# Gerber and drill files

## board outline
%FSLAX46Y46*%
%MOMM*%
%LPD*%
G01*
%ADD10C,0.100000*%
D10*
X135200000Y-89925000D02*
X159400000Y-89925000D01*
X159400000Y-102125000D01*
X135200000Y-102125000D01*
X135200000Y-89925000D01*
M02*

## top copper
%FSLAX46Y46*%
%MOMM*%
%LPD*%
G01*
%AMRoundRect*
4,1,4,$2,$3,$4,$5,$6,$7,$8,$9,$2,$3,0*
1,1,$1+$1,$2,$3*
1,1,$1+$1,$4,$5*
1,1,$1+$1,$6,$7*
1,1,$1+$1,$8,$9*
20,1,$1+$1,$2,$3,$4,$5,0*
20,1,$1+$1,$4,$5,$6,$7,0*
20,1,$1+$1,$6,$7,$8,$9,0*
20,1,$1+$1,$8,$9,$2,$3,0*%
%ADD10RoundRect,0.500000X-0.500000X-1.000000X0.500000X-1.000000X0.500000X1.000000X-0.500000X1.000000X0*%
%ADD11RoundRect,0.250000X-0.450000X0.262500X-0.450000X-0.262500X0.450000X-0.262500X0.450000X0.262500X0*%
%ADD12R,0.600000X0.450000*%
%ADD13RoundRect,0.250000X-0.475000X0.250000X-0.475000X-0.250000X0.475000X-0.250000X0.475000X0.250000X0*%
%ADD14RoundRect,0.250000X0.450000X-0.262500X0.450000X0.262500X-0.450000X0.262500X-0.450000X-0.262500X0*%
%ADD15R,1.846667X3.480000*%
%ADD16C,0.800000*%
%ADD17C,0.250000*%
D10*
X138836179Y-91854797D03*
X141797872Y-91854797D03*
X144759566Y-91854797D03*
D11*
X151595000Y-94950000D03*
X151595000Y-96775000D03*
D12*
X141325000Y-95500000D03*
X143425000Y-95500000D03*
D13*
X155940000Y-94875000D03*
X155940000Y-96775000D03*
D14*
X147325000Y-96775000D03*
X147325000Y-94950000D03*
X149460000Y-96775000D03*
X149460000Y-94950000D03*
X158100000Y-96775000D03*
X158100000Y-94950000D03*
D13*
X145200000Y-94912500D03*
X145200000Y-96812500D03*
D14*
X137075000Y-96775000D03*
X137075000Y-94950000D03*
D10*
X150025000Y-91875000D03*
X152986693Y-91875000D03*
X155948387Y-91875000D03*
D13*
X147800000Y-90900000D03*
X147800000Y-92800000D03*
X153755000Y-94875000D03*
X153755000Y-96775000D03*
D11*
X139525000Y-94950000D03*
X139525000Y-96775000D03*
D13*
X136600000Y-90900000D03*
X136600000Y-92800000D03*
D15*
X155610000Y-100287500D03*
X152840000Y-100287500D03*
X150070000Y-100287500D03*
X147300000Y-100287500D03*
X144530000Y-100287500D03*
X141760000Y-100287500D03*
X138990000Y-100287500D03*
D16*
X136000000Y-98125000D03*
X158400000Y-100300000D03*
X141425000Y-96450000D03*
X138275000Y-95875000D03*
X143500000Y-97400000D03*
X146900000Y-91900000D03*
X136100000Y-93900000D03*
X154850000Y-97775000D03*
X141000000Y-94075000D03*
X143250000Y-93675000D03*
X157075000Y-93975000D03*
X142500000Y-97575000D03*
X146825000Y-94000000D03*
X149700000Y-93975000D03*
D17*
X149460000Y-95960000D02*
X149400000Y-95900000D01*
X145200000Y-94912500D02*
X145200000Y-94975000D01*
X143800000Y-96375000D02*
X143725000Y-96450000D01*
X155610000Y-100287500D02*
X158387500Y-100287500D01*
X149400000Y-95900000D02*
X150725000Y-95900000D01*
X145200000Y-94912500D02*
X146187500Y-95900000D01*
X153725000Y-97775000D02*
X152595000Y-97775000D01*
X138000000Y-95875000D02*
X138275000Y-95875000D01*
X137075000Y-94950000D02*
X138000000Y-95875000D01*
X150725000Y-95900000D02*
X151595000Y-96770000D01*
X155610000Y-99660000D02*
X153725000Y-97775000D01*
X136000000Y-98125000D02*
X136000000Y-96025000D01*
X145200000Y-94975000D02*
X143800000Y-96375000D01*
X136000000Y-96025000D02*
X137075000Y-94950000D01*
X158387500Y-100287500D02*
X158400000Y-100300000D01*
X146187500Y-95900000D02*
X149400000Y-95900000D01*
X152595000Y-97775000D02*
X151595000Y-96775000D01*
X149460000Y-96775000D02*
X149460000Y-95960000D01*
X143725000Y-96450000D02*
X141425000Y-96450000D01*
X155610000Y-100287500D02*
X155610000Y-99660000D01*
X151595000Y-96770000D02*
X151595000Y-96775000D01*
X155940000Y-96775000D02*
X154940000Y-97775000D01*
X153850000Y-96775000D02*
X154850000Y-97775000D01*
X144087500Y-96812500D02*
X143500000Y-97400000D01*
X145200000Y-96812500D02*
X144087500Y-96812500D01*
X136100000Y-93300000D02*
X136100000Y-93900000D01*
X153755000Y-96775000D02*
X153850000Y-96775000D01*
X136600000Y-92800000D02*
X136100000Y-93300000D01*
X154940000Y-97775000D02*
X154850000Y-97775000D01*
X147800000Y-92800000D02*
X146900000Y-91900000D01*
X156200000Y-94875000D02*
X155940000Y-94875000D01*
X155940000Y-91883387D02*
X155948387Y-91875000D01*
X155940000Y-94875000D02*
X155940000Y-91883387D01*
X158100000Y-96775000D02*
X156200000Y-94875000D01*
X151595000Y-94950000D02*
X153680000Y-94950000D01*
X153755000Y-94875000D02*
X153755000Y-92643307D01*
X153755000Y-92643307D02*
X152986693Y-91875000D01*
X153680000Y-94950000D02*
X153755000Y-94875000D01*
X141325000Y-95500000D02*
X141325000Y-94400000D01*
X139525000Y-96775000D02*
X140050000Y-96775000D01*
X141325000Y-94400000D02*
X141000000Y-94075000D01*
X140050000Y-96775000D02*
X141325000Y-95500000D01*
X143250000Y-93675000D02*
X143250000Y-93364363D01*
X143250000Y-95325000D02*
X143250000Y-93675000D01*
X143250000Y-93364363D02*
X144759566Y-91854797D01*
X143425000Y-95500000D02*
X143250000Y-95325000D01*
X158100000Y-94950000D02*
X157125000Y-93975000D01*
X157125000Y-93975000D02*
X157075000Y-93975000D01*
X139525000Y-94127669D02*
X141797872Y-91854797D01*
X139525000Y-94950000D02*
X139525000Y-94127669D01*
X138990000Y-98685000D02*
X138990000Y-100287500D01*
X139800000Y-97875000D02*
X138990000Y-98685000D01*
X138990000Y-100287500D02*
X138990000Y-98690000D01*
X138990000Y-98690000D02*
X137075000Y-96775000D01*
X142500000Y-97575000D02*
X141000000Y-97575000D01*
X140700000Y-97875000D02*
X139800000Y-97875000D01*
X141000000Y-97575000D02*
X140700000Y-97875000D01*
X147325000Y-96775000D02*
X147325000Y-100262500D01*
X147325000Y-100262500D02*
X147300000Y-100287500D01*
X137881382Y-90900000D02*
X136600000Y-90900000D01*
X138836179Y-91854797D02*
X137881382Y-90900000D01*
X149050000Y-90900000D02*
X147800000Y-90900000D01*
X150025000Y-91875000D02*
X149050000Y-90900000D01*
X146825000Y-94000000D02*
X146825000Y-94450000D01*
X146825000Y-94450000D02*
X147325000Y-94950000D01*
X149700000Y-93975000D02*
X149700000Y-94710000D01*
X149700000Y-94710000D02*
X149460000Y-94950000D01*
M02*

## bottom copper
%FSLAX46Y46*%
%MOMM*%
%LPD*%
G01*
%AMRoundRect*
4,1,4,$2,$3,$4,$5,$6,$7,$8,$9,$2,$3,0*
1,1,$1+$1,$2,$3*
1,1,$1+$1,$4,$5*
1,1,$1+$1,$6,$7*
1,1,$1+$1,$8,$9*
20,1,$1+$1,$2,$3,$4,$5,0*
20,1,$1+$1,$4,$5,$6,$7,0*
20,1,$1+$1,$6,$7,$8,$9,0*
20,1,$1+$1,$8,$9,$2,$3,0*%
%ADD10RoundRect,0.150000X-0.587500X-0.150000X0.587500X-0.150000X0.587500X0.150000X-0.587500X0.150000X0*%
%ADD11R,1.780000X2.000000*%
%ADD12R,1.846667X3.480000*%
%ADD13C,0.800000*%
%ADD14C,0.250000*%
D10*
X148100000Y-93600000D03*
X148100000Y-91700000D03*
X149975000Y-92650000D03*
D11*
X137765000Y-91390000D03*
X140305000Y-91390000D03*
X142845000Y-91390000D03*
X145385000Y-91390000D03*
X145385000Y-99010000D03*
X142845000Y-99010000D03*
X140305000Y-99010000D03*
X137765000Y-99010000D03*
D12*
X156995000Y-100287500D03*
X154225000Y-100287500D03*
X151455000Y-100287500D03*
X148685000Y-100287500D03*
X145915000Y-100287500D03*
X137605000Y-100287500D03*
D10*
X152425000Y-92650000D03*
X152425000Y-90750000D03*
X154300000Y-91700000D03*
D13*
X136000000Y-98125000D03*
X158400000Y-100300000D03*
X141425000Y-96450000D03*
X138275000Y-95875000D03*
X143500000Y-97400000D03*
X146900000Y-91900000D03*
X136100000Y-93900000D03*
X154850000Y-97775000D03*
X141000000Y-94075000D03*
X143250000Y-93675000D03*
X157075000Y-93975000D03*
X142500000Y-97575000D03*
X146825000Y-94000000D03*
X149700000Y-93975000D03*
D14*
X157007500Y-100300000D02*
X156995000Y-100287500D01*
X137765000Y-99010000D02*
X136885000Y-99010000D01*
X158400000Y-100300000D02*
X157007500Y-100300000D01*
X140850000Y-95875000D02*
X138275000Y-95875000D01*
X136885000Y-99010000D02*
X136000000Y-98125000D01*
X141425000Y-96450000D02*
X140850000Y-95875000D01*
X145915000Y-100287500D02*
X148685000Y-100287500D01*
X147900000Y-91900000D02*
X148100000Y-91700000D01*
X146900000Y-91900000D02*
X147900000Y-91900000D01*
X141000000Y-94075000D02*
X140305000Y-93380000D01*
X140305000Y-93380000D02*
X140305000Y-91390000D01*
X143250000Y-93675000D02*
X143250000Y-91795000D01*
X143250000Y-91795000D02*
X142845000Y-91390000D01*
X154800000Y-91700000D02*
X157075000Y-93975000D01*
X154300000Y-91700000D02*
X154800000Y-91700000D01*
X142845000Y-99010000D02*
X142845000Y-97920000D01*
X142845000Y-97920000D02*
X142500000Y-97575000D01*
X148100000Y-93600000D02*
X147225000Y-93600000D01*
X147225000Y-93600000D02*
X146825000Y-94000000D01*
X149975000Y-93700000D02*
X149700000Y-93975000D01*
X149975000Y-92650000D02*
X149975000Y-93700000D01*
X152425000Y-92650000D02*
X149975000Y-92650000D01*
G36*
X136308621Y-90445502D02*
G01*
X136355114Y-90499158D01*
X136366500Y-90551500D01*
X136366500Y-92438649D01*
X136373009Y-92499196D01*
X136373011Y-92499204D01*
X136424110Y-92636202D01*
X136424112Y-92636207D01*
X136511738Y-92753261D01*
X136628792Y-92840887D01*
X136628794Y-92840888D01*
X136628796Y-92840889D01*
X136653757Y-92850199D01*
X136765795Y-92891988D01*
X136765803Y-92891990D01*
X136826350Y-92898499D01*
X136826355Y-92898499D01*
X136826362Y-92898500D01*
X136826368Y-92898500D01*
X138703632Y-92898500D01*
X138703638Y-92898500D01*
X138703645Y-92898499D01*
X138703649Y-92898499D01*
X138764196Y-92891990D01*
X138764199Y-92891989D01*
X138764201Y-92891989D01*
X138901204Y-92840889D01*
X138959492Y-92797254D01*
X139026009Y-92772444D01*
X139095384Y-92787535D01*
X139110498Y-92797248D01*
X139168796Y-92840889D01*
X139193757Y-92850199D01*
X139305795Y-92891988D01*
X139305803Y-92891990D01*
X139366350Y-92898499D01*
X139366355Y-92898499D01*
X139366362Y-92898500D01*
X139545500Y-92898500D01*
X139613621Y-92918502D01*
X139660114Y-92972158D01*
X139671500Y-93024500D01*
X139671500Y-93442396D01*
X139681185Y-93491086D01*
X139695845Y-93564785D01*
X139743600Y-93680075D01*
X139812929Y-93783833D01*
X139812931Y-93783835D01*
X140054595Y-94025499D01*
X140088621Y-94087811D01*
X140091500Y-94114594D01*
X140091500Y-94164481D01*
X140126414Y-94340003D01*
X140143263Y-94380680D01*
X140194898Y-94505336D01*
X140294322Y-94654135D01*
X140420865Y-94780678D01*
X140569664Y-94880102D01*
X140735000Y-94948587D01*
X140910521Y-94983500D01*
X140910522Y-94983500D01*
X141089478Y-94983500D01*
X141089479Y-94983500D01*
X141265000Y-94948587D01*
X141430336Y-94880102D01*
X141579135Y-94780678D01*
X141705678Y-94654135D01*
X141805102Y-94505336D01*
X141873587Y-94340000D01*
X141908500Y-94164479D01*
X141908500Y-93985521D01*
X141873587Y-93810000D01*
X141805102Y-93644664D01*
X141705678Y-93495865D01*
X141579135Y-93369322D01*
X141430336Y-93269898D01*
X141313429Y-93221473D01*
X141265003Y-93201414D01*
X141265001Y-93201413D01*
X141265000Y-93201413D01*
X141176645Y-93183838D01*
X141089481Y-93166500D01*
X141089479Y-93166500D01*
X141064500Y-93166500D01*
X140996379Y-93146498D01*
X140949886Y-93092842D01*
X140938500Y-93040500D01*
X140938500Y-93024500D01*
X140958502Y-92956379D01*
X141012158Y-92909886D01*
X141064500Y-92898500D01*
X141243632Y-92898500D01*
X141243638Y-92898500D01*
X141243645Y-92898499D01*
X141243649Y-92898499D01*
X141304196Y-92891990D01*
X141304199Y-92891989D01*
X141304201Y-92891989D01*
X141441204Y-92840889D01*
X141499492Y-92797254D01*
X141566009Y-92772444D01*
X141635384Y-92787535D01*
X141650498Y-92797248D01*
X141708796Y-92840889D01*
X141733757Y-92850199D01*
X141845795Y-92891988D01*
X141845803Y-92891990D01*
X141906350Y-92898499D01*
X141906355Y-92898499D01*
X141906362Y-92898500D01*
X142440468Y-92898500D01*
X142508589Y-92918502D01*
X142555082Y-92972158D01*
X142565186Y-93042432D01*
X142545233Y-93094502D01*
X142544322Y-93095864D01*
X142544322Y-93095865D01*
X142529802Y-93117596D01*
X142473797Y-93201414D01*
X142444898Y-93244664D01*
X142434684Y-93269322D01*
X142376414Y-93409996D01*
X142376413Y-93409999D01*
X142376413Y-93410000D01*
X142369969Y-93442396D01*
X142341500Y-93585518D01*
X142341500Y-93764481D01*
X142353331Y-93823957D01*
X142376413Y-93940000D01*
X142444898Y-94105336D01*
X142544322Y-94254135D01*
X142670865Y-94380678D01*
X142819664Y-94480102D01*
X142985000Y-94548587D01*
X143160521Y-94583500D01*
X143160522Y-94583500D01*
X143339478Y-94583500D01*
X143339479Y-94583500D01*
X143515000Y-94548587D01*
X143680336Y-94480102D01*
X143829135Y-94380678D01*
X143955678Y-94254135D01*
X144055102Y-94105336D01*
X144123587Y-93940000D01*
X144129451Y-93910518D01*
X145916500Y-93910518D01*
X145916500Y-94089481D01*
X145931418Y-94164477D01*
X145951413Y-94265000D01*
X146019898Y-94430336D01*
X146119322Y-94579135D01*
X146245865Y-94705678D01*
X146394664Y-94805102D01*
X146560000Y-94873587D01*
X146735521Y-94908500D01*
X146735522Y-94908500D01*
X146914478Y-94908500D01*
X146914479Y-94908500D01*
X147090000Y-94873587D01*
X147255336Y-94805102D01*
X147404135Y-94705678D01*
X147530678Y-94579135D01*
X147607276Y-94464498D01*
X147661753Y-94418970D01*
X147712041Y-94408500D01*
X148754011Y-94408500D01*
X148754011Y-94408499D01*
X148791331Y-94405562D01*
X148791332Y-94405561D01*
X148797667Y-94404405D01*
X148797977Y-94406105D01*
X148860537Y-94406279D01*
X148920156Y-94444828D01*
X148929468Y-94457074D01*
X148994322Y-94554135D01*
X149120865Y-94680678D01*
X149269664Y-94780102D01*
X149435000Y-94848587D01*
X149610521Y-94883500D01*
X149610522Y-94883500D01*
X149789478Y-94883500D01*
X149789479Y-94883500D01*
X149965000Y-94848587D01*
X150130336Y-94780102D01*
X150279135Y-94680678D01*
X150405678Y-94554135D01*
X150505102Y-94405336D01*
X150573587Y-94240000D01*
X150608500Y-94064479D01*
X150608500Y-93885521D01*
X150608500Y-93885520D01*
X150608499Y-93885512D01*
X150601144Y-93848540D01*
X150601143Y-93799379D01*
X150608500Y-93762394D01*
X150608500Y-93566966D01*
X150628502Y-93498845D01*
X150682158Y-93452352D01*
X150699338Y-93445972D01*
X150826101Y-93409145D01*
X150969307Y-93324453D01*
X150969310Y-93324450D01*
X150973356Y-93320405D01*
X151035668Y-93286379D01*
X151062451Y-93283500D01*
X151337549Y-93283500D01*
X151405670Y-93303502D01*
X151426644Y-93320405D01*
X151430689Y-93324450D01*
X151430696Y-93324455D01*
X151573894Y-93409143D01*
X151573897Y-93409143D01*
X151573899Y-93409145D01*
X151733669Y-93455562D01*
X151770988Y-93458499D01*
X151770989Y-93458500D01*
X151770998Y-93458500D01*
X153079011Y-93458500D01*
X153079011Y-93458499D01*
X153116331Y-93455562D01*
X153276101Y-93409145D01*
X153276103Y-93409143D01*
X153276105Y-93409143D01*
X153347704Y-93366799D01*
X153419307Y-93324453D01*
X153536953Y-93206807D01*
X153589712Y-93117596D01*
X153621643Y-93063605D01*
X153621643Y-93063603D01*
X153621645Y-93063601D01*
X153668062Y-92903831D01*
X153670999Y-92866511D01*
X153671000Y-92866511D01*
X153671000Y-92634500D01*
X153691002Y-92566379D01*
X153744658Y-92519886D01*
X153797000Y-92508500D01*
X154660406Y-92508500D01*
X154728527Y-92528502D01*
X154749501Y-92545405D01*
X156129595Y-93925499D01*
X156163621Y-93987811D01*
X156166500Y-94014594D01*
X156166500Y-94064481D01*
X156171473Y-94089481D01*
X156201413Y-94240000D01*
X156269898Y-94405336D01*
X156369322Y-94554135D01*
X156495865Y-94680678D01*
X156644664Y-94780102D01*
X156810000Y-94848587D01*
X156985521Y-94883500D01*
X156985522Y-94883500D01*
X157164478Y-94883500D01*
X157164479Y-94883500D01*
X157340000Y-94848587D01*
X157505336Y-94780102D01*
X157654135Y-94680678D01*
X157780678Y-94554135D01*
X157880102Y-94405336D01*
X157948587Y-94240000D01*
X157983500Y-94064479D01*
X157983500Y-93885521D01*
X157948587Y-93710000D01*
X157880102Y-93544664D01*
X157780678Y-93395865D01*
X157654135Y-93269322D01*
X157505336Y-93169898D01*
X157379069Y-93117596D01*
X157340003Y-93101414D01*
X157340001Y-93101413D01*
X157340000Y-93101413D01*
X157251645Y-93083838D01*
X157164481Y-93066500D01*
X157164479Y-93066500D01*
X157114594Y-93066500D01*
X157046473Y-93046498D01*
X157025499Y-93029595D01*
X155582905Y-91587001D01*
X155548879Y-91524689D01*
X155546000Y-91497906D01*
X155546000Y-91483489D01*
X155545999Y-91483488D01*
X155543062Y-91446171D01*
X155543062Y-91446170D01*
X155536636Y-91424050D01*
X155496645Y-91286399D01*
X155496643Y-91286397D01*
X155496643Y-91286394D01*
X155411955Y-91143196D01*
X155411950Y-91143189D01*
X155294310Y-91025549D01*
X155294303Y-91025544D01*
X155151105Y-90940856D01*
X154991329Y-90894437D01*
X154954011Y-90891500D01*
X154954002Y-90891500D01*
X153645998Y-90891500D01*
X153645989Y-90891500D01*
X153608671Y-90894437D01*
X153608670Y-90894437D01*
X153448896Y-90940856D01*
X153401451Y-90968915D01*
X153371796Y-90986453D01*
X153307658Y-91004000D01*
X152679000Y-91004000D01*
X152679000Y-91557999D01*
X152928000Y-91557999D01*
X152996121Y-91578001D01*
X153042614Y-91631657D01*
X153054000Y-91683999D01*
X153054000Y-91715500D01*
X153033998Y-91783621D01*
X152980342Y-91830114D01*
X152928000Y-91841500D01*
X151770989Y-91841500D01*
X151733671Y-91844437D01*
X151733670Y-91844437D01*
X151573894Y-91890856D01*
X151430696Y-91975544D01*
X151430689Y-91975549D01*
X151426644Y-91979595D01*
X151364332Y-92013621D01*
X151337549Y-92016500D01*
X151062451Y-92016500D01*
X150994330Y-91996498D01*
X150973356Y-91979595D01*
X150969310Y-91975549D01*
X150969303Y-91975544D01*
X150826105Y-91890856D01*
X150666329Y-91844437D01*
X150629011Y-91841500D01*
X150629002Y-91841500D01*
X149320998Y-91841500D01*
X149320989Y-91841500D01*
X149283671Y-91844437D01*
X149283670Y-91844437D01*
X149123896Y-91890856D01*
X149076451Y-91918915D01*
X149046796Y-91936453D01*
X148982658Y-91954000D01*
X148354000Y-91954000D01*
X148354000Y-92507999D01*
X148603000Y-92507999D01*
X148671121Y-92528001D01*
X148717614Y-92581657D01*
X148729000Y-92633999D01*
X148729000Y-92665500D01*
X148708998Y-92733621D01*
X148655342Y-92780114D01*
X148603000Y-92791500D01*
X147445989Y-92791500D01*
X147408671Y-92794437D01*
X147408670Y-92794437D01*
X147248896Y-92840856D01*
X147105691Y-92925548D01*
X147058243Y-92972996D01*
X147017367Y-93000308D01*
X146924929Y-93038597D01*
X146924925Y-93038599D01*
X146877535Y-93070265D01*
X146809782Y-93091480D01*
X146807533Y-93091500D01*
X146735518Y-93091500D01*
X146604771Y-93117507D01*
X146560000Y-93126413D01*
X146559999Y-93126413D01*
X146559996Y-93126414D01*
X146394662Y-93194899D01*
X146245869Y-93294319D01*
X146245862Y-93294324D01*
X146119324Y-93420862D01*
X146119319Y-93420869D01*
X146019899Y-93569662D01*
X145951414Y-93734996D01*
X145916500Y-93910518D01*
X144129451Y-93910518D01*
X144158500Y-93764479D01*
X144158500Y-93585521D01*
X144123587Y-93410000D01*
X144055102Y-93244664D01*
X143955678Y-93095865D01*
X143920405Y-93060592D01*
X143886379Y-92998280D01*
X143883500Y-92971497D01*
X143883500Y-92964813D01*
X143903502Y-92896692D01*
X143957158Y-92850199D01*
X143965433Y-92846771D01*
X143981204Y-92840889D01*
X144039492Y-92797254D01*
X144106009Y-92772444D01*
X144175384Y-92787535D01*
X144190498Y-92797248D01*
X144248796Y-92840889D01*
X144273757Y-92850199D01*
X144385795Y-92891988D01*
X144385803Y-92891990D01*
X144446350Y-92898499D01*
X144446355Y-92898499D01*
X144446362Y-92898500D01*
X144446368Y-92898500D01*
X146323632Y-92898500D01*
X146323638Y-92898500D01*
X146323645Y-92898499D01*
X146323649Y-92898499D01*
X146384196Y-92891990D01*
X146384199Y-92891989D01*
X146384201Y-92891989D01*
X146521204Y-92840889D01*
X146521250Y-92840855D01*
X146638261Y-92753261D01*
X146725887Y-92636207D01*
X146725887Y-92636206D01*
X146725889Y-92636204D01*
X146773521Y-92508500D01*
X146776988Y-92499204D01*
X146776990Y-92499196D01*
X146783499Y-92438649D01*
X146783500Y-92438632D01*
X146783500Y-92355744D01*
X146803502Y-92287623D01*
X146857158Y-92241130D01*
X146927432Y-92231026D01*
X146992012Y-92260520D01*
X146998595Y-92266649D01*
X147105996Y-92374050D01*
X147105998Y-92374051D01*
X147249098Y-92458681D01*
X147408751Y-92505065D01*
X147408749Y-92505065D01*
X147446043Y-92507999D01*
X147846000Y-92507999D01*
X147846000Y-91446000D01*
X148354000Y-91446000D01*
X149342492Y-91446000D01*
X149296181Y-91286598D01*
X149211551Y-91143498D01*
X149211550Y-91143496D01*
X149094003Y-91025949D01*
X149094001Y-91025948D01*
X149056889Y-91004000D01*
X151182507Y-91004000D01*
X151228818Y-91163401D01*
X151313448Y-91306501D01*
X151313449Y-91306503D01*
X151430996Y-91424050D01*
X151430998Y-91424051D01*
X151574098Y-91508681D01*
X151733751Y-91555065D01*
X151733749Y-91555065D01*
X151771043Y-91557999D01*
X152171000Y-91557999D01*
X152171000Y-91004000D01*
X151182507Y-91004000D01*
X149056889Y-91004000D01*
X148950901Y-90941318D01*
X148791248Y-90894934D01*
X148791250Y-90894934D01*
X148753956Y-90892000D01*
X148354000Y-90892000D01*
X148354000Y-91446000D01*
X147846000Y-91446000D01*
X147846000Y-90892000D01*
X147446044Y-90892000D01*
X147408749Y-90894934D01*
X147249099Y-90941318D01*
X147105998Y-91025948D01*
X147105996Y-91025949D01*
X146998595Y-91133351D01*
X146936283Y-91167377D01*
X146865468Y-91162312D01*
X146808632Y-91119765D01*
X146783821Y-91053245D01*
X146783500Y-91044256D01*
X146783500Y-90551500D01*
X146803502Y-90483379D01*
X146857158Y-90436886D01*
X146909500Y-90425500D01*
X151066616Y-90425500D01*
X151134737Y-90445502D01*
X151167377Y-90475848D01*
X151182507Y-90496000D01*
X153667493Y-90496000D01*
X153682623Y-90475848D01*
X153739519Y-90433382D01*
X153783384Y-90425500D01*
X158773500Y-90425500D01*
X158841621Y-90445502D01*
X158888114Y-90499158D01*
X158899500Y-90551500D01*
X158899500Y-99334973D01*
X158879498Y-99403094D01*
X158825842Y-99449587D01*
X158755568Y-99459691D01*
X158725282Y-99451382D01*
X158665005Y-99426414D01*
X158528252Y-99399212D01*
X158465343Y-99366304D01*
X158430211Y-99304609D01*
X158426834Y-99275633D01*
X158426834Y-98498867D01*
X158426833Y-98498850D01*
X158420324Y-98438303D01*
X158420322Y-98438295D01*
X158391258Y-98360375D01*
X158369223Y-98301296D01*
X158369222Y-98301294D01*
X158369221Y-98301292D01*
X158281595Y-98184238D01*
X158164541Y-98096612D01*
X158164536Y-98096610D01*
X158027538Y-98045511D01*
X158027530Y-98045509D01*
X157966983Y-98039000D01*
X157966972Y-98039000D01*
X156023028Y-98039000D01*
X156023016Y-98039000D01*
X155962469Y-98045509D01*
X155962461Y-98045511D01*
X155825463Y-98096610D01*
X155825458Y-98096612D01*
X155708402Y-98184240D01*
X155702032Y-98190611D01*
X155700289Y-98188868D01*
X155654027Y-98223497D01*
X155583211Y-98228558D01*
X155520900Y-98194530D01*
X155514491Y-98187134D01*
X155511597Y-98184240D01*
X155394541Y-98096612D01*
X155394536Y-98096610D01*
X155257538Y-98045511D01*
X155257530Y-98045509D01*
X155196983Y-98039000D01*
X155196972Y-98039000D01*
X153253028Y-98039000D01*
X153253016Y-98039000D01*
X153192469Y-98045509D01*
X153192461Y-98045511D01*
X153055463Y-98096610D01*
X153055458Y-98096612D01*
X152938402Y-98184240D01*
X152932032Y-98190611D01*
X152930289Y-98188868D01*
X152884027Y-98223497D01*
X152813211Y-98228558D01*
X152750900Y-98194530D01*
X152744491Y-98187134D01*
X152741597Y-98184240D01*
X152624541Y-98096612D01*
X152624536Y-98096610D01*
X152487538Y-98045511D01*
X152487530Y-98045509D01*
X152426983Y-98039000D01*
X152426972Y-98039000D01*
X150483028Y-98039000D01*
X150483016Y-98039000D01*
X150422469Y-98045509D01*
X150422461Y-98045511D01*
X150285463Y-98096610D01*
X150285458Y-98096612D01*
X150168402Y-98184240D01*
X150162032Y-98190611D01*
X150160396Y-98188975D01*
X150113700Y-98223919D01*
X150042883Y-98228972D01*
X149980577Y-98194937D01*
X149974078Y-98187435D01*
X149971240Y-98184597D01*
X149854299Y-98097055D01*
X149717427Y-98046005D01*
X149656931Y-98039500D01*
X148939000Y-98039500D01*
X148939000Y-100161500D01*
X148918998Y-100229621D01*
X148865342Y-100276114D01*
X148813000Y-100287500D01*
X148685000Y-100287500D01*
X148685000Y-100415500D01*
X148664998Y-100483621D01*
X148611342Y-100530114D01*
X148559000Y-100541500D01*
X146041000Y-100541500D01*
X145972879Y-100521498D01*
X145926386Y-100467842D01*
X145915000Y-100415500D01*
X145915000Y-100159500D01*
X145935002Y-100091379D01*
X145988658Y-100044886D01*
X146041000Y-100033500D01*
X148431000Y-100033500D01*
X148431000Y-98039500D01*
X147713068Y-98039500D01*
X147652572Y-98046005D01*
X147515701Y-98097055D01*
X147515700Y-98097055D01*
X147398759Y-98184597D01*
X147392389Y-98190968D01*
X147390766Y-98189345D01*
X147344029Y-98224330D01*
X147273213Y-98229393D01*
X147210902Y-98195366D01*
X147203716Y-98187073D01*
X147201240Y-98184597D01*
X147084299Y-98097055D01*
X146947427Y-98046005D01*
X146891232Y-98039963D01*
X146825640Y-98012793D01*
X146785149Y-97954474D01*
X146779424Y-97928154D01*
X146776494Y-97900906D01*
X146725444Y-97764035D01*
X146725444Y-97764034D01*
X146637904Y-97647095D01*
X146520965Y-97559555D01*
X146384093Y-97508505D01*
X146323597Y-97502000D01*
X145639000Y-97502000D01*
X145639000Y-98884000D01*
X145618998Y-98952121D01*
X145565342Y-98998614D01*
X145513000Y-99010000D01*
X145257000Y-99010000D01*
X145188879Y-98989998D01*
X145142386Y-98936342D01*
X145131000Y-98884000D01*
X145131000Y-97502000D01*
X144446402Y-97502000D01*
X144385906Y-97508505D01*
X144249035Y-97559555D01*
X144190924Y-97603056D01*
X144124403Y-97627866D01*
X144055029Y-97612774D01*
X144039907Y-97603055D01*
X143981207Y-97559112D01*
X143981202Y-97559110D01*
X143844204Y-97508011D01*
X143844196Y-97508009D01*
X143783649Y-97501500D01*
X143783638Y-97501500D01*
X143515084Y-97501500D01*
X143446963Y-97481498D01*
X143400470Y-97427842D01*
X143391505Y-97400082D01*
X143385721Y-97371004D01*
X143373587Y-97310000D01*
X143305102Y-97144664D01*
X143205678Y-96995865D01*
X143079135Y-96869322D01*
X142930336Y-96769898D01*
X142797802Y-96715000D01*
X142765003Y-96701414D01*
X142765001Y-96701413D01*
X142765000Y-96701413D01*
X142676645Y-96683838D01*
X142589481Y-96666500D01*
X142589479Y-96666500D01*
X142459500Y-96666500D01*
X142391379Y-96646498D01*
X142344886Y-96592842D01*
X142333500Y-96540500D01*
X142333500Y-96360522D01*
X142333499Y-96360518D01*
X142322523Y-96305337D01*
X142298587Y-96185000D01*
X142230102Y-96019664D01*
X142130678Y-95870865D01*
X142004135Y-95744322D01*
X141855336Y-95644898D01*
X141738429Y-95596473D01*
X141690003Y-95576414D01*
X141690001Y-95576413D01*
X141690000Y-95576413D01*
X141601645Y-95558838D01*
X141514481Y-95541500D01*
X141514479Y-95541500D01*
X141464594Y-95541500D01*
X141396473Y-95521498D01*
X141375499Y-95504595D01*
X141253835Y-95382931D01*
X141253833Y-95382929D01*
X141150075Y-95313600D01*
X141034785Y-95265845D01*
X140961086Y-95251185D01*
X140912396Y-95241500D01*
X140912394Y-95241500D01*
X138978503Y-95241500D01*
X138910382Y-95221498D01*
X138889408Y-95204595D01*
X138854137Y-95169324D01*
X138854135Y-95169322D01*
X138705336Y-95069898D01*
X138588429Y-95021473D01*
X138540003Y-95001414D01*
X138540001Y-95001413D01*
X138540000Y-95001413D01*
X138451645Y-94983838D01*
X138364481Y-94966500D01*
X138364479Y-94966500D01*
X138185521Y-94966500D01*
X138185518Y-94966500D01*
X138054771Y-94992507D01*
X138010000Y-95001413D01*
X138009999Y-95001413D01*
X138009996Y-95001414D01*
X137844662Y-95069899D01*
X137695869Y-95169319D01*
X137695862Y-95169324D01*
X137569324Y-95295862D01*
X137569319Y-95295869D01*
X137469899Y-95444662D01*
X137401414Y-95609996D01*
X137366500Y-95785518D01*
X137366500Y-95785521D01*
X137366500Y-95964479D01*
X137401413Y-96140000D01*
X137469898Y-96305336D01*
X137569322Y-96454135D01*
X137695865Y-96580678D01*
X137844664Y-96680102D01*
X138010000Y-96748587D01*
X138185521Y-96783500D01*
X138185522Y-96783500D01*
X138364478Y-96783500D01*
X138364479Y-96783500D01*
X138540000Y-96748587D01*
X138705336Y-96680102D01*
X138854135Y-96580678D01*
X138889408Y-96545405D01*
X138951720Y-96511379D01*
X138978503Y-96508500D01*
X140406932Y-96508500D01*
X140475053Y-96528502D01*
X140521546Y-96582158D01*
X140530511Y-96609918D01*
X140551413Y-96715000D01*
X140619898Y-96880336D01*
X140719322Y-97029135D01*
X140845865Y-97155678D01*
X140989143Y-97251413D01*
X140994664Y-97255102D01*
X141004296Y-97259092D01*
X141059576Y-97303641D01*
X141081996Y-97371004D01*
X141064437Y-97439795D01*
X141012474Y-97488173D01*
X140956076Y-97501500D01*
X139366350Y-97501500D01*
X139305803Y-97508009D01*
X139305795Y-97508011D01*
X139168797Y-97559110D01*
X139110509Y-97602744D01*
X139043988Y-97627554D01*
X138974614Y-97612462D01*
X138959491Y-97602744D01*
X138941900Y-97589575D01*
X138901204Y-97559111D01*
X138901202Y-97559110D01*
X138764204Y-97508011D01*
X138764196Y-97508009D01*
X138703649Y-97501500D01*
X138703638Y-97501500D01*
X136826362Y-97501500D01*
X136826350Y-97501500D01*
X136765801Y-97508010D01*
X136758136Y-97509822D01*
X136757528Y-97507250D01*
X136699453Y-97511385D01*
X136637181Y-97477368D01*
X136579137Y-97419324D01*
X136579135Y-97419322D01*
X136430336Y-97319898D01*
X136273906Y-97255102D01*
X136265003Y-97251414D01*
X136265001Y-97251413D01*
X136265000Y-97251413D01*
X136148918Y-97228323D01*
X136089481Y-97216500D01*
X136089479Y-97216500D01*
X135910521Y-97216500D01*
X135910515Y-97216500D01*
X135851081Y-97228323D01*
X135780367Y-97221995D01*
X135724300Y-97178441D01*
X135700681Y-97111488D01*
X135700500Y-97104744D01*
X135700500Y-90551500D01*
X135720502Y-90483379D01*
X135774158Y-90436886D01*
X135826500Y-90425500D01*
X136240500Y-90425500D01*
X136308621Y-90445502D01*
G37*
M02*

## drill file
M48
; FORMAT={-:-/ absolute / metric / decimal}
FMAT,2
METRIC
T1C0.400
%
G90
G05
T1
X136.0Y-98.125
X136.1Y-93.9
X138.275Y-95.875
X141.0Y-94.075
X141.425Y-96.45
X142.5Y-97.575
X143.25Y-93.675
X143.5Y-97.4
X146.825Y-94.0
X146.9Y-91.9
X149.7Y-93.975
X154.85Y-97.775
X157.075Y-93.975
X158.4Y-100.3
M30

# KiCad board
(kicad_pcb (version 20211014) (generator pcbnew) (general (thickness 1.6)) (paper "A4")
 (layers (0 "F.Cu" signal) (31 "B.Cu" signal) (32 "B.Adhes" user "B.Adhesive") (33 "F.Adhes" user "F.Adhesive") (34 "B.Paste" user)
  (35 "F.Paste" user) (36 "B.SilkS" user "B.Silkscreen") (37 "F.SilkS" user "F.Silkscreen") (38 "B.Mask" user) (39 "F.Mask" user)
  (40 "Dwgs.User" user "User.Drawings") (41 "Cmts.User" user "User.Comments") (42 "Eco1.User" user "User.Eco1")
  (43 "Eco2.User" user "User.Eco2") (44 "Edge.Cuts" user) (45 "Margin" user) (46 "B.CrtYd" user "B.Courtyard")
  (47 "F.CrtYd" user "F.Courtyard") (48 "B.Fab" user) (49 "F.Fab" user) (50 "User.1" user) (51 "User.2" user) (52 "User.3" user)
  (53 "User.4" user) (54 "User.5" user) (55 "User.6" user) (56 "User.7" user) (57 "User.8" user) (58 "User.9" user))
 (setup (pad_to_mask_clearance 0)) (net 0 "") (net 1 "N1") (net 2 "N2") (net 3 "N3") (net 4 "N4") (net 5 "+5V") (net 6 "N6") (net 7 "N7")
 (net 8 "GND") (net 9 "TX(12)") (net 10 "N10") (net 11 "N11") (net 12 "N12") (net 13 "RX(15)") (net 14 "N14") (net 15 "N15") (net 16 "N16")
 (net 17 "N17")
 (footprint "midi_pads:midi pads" (layer "F.Cu") (at 141.9 95.225)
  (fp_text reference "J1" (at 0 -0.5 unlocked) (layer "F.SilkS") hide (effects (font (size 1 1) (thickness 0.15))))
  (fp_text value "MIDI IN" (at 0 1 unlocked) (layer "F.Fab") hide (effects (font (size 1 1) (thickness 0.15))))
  (pad "2" smd roundrect (at -3.063821 -3.370203) (size 2 3) (layers "F.Cu" "F.Paste" "F.Mask") (roundrect_rratio 0.25) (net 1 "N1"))
  (pad "4" smd roundrect (at -0.102128 -3.370203) (size 2 3) (layers "F.Cu" "F.Paste" "F.Mask") (roundrect_rratio 0.25) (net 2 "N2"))
  (pad "5" smd roundrect (at 2.859566 -3.370203) (size 2 3) (layers "F.Cu" "F.Paste" "F.Mask") (roundrect_rratio 0.25) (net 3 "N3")))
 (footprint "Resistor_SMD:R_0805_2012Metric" (layer "F.Cu") (at 151.595 95.8625 -90)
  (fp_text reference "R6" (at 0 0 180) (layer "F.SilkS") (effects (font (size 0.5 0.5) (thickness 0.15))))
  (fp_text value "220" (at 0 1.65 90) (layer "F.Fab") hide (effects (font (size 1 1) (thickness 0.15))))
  (pad "1" smd roundrect (at -0.9125 0 270) (size 1.025 1.4) (layers "F.Cu" "F.Paste" "F.Mask") (roundrect_rratio 0.243902439) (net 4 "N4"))
  (pad "2" smd roundrect (at 0.9125 0 270) (size 1.025 1.4) (layers "F.Cu" "F.Paste" "F.Mask") (roundrect_rratio 0.243902439) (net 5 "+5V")))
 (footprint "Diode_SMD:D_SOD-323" (layer "F.Cu") (at 142.375 95.5)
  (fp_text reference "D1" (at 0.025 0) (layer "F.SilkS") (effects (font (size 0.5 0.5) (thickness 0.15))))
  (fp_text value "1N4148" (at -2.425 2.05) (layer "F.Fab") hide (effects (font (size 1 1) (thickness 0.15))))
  (pad "1" smd rect (at -1.05 0) (size 0.6 0.45) (layers "F.Cu" "F.Paste" "F.Mask") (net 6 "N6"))
  (pad "2" smd rect (at 1.05 0) (size 0.6 0.45) (layers "F.Cu" "F.Paste" "F.Mask") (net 3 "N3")))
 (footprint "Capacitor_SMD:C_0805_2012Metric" (layer "F.Cu") (at 155.94 95.825 -90)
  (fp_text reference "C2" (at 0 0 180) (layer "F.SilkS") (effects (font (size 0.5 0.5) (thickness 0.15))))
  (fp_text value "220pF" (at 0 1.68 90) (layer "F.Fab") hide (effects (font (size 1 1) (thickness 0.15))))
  (pad "1" smd roundrect (at -0.95 0 270) (size 1 1.45) (layers "F.Cu" "F.Paste" "F.Mask") (roundrect_rratio 0.25) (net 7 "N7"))
  (pad "2" smd roundrect (at 0.95 0 270) (size 1 1.45) (layers "F.Cu" "F.Paste" "F.Mask") (roundrect_rratio 0.25) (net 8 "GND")))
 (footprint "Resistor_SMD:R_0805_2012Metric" (layer "F.Cu") (at 147.325 95.8625 90)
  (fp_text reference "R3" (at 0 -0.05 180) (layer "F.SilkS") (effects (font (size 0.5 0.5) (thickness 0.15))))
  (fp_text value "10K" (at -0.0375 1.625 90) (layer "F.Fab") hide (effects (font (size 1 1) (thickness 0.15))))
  (pad "1" smd roundrect (at -0.9125 0 90) (size 1.025 1.4) (layers "F.Cu" "F.Paste" "F.Mask") (roundrect_rratio 0.243902439)
   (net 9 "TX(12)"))
  (pad "2" smd roundrect (at 0.9125 0 90) (size 1.025 1.4) (layers "F.Cu" "F.Paste" "F.Mask") (roundrect_rratio 0.243902439) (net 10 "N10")))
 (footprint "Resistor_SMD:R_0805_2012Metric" (layer "F.Cu") (at 149.46 95.8625 90)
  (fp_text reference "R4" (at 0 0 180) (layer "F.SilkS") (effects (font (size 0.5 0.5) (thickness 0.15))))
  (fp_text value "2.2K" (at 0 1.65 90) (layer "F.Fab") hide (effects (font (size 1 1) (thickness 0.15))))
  (pad "1" smd roundrect (at -0.9125 0 90) (size 1.025 1.4) (layers "F.Cu" "F.Paste" "F.Mask") (roundrect_rratio 0.243902439) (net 5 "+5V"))
  (pad "2" smd roundrect (at 0.9125 0 90) (size 1.025 1.4) (layers "F.Cu" "F.Paste" "F.Mask") (roundrect_rratio 0.243902439) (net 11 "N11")))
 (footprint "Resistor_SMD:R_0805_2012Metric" (layer "F.Cu") (at 158.1 95.8625 90)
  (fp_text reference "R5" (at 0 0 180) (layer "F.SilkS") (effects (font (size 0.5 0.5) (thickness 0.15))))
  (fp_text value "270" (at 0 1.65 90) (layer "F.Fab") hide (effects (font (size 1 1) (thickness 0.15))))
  (pad "1" smd roundrect (at -0.9125 0 90) (size 1.025 1.4) (layers "F.Cu" "F.Paste" "F.Mask") (roundrect_rratio 0.243902439) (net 7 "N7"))
  (pad "2" smd roundrect (at 0.9125 0 90) (size 1.025 1.4) (layers "F.Cu" "F.Paste" "F.Mask") (roundrect_rratio 0.243902439) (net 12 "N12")))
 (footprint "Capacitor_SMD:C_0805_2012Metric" (layer "F.Cu") (at 145.2 95.8625 -90)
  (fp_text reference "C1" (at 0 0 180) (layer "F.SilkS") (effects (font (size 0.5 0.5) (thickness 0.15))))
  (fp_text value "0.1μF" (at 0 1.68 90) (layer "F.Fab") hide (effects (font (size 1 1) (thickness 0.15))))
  (pad "1" smd roundrect (at -0.95 0 270) (size 1 1.45) (layers "F.Cu" "F.Paste" "F.Mask") (roundrect_rratio 0.25) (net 5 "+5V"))
  (pad "2" smd roundrect (at 0.95 0 270) (size 1 1.45) (layers "F.Cu" "F.Paste" "F.Mask") (roundrect_rratio 0.25) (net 8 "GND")))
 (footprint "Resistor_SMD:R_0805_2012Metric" (layer "F.Cu") (at 137.075 95.8625 90)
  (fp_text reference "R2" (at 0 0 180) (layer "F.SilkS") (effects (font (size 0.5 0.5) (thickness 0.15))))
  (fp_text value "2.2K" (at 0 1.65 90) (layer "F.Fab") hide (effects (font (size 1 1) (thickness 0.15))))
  (pad "1" smd roundrect (at -0.9125 0 90) (size 1.025 1.4) (layers "F.Cu" "F.Paste" "F.Mask") (roundrect_rratio 0.243902439)
   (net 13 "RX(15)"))
  (pad "2" smd roundrect (at 0.9125 0 90) (size 1.025 1.4) (layers "F.Cu" "F.Paste" "F.Mask") (roundrect_rratio 0.243902439) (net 5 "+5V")))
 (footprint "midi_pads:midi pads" (layer "F.Cu") (at 153.088821 95.245203)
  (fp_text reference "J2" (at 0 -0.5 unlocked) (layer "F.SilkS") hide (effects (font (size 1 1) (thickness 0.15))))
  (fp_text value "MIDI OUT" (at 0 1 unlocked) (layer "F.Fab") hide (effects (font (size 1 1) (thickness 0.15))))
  (pad "2" smd roundrect (at -3.063821 -3.370203) (size 2 3) (layers "F.Cu" "F.Paste" "F.Mask") (roundrect_rratio 0.25) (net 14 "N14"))
  (pad "4" smd roundrect (at -0.102128 -3.370203) (size 2 3) (layers "F.Cu" "F.Paste" "F.Mask") (roundrect_rratio 0.25) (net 4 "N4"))
  (pad "5" smd roundrect (at 2.859566 -3.370203) (size 2 3) (layers "F.Cu" "F.Paste" "F.Mask") (roundrect_rratio 0.25) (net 7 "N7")))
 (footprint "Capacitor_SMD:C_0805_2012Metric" (layer "F.Cu") (at 147.8 91.85 -90)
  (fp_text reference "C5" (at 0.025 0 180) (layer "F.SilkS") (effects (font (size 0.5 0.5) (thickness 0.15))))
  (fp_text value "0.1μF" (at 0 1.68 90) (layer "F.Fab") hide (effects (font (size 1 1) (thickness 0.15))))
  (pad "1" smd roundrect (at -0.95 0 270) (size 1 1.45) (layers "F.Cu" "F.Paste" "F.Mask") (roundrect_rratio 0.25) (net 14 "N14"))
  (pad "2" smd roundrect (at 0.95 0 270) (size 1 1.45) (layers "F.Cu" "F.Paste" "F.Mask") (roundrect_rratio 0.25) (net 8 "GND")))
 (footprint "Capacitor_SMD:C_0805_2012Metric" (layer "F.Cu") (at 153.755 95.825 -90)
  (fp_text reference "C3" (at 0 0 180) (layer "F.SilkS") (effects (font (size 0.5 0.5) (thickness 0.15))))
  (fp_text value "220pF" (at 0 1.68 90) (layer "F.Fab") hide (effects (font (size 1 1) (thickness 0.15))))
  (pad "1" smd roundrect (at -0.95 0 270) (size 1 1.45) (layers "F.Cu" "F.Paste" "F.Mask") (roundrect_rratio 0.25) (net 4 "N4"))
  (pad "2" smd roundrect (at 0.95 0 270) (size 1 1.45) (layers "F.Cu" "F.Paste" "F.Mask") (roundrect_rratio 0.25) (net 8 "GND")))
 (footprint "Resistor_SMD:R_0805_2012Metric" (layer "F.Cu") (at 139.525 95.8625 -90)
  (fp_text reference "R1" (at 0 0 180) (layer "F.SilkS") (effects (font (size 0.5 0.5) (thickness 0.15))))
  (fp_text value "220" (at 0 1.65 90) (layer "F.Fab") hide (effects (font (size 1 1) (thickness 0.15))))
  (pad "1" smd roundrect (at -0.9125 0 270) (size 1.025 1.4) (layers "F.Cu" "F.Paste" "F.Mask") (roundrect_rratio 0.243902439) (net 2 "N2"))
  (pad "2" smd roundrect (at 0.9125 0 270) (size 1.025 1.4) (layers "F.Cu" "F.Paste" "F.Mask") (roundrect_rratio 0.243902439) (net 6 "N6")))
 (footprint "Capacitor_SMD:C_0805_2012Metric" (layer "F.Cu") (at 136.6 91.85 -90)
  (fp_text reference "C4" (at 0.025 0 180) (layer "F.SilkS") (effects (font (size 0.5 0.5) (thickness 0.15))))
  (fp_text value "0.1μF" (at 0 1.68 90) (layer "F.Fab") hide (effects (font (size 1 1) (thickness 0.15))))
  (pad "1" smd roundrect (at -0.95 0 270) (size 1 1.45) (layers "F.Cu" "F.Paste" "F.Mask") (roundrect_rratio 0.25) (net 1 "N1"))
  (pad "2" smd roundrect (at 0.95 0 270) (size 1 1.45) (layers "F.Cu" "F.Paste" "F.Mask") (roundrect_rratio 0.25) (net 8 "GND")))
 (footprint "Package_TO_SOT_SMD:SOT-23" (layer "B.Cu") (at 149.0375 92.65)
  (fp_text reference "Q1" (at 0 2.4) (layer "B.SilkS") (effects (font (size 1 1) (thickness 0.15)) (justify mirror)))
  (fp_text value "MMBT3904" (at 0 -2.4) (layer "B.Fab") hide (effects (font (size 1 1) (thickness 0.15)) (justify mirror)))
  (pad "1" smd roundrect (at -0.9375 0.95) (size 1.475 0.6) (layers "B.Cu" "B.Paste" "B.Mask") (roundrect_rratio 0.25) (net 10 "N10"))
  (pad "2" smd roundrect (at -0.9375 -0.95) (size 1.475 0.6) (layers "B.Cu" "B.Paste" "B.Mask") (roundrect_rratio 0.25) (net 8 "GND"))
  (pad "3" smd roundrect (at 0.9375 0) (size 1.475 0.6) (layers "B.Cu" "B.Paste" "B.Mask") (roundrect_rratio 0.25) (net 11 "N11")))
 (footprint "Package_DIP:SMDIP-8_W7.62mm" (layer "B.Cu") (at 141.575 95.2 -90)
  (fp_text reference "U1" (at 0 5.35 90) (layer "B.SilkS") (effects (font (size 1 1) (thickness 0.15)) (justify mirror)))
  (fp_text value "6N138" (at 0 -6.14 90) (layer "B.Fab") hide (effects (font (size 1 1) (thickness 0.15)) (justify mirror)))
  (pad "1" smd rect (at -3.81 3.81 270) (size 2 1.78) (layers "B.Cu" "B.Paste" "B.Mask") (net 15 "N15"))
  (pad "2" smd rect (at -3.81 1.27 270) (size 2 1.78) (layers "B.Cu" "B.Paste" "B.Mask") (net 6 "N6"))
  (pad "3" smd rect (at -3.81 -1.27 270) (size 2 1.78) (layers "B.Cu" "B.Paste" "B.Mask") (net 3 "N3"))
  (pad "4" smd rect (at -3.81 -3.81 270) (size 2 1.78) (layers "B.Cu" "B.Paste" "B.Mask") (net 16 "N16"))
  (pad "5" smd rect (at 3.81 -3.81 270) (size 2 1.78) (layers "B.Cu" "B.Paste" "B.Mask") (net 8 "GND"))
  (pad "6" smd rect (at 3.81 -1.27 270) (size 2 1.78) (layers "B.Cu" "B.Paste" "B.Mask") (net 13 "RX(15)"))
  (pad "7" smd rect (at 3.81 1.27 270) (size 2 1.78) (layers "B.Cu" "B.Paste" "B.Mask") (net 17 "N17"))
  (pad "8" smd rect (at 3.81 3.81 270) (size 2 1.78) (layers "B.Cu" "B.Paste" "B.Mask") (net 5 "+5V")))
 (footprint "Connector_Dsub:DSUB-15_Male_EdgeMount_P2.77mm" (layer "B.Cu") (at 147.3 100.2875 180)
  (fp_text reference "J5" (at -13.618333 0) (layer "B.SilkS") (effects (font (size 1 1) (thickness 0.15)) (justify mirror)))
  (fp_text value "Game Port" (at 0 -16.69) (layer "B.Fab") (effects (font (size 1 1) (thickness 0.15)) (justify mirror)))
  (pad "1" smd rect (at -9.695 0 180) (size 1.846667 3.48) (layers "B.Cu" "B.Paste" "B.Mask") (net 5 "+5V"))
  (pad "2" smd rect (at -6.925 0 180) (size 1.846667 3.48) (layers "B.Cu" "B.Paste" "B.Mask"))
  (pad "3" smd rect (at -4.155 0 180) (size 1.846667 3.48) (layers "B.Cu" "B.Paste" "B.Mask"))
  (pad "4" smd rect (at -1.385 0 180) (size 1.846667 3.48) (layers "B.Cu" "B.Paste" "B.Mask") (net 8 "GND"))
  (pad "5" smd rect (at 1.385 0 180) (size 1.846667 3.48) (layers "B.Cu" "B.Paste" "B.Mask") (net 8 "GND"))
  (pad "8" smd rect (at 9.695 0 180) (size 1.846667 3.48) (layers "B.Cu" "B.Paste" "B.Mask") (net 5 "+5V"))
  (pad "9" smd rect (at -8.31 0 180) (size 1.846667 3.48) (layers "F.Cu" "F.Paste" "F.Mask") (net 5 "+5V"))
  (pad "10" smd rect (at -5.54 0 180) (size 1.846667 3.48) (layers "F.Cu" "F.Paste" "F.Mask"))
  (pad "11" smd rect (at -2.77 0 180) (size 1.846667 3.48) (layers "F.Cu" "F.Paste" "F.Mask"))
  (pad "12" smd rect (at 0 0 180) (size 1.846667 3.48) (layers "F.Cu" "F.Paste" "F.Mask") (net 9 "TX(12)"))
  (pad "13" smd rect (at 2.77 0 180) (size 1.846667 3.48) (layers "F.Cu" "F.Paste" "F.Mask"))
  (pad "14" smd rect (at 5.54 0 180) (size 1.846667 3.48) (layers "F.Cu" "F.Paste" "F.Mask"))
  (pad "15" smd rect (at 8.31 0 180) (size 1.846667 3.48) (layers "F.Cu" "F.Paste" "F.Mask") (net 13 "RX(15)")))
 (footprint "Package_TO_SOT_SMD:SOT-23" (layer "B.Cu") (at 153.3625 91.7)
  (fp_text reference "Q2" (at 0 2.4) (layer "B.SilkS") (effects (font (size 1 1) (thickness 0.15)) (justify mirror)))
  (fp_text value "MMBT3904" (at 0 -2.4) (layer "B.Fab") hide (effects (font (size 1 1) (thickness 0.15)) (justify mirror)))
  (pad "1" smd roundrect (at -0.9375 0.95) (size 1.475 0.6) (layers "B.Cu" "B.Paste" "B.Mask") (roundrect_rratio 0.25) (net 11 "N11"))
  (pad "2" smd roundrect (at -0.9375 -0.95) (size 1.475 0.6) (layers "B.Cu" "B.Paste" "B.Mask") (roundrect_rratio 0.25) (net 8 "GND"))
  (pad "3" smd roundrect (at 0.9375 0) (size 1.475 0.6) (layers "B.Cu" "B.Paste" "B.Mask") (roundrect_rratio 0.25) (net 12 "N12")))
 (gr_rect (start 159.4 89.925) (end 135.2 102.125) (layer "Edge.Cuts") (width 0.1) (fill none))
 (segment (start 149.46 95.96) (end 149.4 95.9) (width 0.25) (layer "F.Cu") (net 5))
 (segment (start 145.2 94.9125) (end 145.2 94.975) (width 0.25) (layer "F.Cu") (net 5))
 (segment (start 143.8 96.375) (end 143.725 96.45) (width 0.25) (layer "F.Cu") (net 5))
 (segment (start 155.61 100.2875) (end 158.3875 100.2875) (width 0.25) (layer "F.Cu") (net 5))
 (segment (start 149.4 95.9) (end 150.725 95.9) (width 0.25) (layer "F.Cu") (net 5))
 (segment (start 145.2 94.9125) (end 146.1875 95.9) (width 0.25) (layer "F.Cu") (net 5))
 (segment (start 153.725 97.775) (end 152.595 97.775) (width 0.25) (layer "F.Cu") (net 5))
 (segment (start 138 95.875) (end 138.275 95.875) (width 0.25) (layer "F.Cu") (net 5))
 (segment (start 137.075 94.95) (end 138 95.875) (width 0.25) (layer "F.Cu") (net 5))
 (segment (start 150.725 95.9) (end 151.595 96.77) (width 0.25) (layer "F.Cu") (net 5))
 (segment (start 155.61 99.66) (end 153.725 97.775) (width 0.25) (layer "F.Cu") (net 5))
 (segment (start 136 98.125) (end 136 96.025) (width 0.25) (layer "F.Cu") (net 5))
 (segment (start 145.2 94.975) (end 143.8 96.375) (width 0.25) (layer "F.Cu") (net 5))
 (segment (start 136 96.025) (end 137.075 94.95) (width 0.25) (layer "F.Cu") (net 5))
 (segment (start 158.3875 100.2875) (end 158.4 100.3) (width 0.25) (layer "F.Cu") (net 5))
 (segment (start 146.1875 95.9) (end 149.4 95.9) (width 0.25) (layer "F.Cu") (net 5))
 (segment (start 152.595 97.775) (end 151.595 96.775) (width 0.25) (layer "F.Cu") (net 5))
 (segment (start 149.46 96.775) (end 149.46 95.96) (width 0.25) (layer "F.Cu") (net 5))
 (segment (start 143.725 96.45) (end 141.425 96.45) (width 0.25) (layer "F.Cu") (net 5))
 (segment (start 155.61 100.2875) (end 155.61 99.66) (width 0.25) (layer "F.Cu") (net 5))
 (segment (start 151.595 96.77) (end 151.595 96.775) (width 0.25) (layer "F.Cu") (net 5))
 (via (at 136 98.125) (size 0.8) (drill 0.4) (layers "F.Cu" "B.Cu") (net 5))
 (via (at 158.4 100.3) (size 0.8) (drill 0.4) (layers "F.Cu" "B.Cu") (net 5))
 (via (at 141.425 96.45) (size 0.8) (drill 0.4) (layers "F.Cu" "B.Cu") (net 5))
 (via (at 138.275 95.875) (size 0.8) (drill 0.4) (layers "F.Cu" "B.Cu") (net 5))
 (segment (start 157.0075 100.3) (end 156.995 100.2875) (width 0.25) (layer "B.Cu") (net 5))
 (segment (start 137.765 99.01) (end 136.885 99.01) (width 0.25) (layer "B.Cu") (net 5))
 (segment (start 158.4 100.3) (end 157.0075 100.3) (width 0.25) (layer "B.Cu") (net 5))
 (segment (start 140.85 95.875) (end 138.275 95.875) (width 0.25) (layer "B.Cu") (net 5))
 (segment (start 136.885 99.01) (end 136 98.125) (width 0.25) (layer "B.Cu") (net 5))
 (segment (start 141.425 96.45) (end 140.85 95.875) (width 0.25) (layer "B.Cu") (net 5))
 (segment (start 155.94 96.775) (end 154.94 97.775) (width 0.25) (layer "F.Cu") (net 8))
 (segment (start 153.85 96.775) (end 154.85 97.775) (width 0.25) (layer "F.Cu") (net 8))
 (segment (start 144.0875 96.8125) (end 143.5 97.4) (width 0.25) (layer "F.Cu") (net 8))
 (segment (start 145.2 96.8125) (end 144.0875 96.8125) (width 0.25) (layer "F.Cu") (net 8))
 (segment (start 136.1 93.3) (end 136.1 93.9) (width 0.25) (layer "F.Cu") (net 8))
 (segment (start 153.755 96.775) (end 153.85 96.775) (width 0.25) (layer "F.Cu") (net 8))
 (segment (start 136.6 92.8) (end 136.1 93.3) (width 0.25) (layer "F.Cu") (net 8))
 (segment (start 154.94 97.775) (end 154.85 97.775) (width 0.25) (layer "F.Cu") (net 8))
 (segment (start 147.8 92.8) (end 146.9 91.9) (width 0.25) (layer "F.Cu") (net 8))
 (via (at 143.5 97.4) (size 0.8) (drill 0.4) (layers "F.Cu" "B.Cu") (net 8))
 (via (at 146.9 91.9) (size 0.8) (drill 0.4) (layers "F.Cu" "B.Cu") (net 8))
 (via (at 136.1 93.9) (size 0.8) (drill 0.4) (layers "F.Cu" "B.Cu") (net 8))
 (via (at 154.85 97.775) (size 0.8) (drill 0.4) (layers "F.Cu" "B.Cu") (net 8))
 (segment (start 145.915 100.2875) (end 148.685 100.2875) (width 0.25) (layer "B.Cu") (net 8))
 (segment (start 147.9 91.9) (end 148.1 91.7) (width 0.25) (layer "B.Cu") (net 8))
 (segment (start 146.9 91.9) (end 147.9 91.9) (width 0.25) (layer "B.Cu") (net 8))
 (segment (start 156.2 94.875) (end 155.94 94.875) (width 0.25) (layer "F.Cu") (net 7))
 (segment (start 155.94 91.883387) (end 155.948387 91.875) (width 0.25) (layer "F.Cu") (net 7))
 (segment (start 155.94 94.875) (end 155.94 91.883387) (width 0.25) (layer "F.Cu") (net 7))
 (segment (start 158.1 96.775) (end 156.2 94.875) (width 0.25) (layer "F.Cu") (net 7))
 (segment (start 151.595 94.95) (end 153.68 94.95) (width 0.25) (layer "F.Cu") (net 4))
 (segment (start 153.755 94.875) (end 153.755 92.643307) (width 0.25) (layer "F.Cu") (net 4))
 (segment (start 153.755 92.643307) (end 152.986693 91.875) (width 0.25) (layer "F.Cu") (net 4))
 (segment (start 153.68 94.95) (end 153.755 94.875) (width 0.25) (layer "F.Cu") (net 4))
 (segment (start 141.325 95.5) (end 141.325 94.4) (width 0.25) (layer "F.Cu") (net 6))
 (segment (start 139.525 96.775) (end 140.05 96.775) (width 0.25) (layer "F.Cu") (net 6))
 (segment (start 141.325 94.4) (end 141 94.075) (width 0.25) (layer "F.Cu") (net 6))
 (segment (start 140.05 96.775) (end 141.325 95.5) (width 0.25) (layer "F.Cu") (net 6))
 (via (at 141 94.075) (size 0.8) (drill 0.4) (layers "F.Cu" "B.Cu") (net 6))
 (segment (start 141 94.075) (end 140.305 93.38) (width 0.25) (layer "B.Cu") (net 6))
 (segment (start 140.305 93.38) (end 140.305 91.39) (width 0.25) (layer "B.Cu") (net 6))
 (segment (start 143.25 93.675) (end 143.25 93.364363) (width 0.25) (layer "F.Cu") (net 3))
 (segment (start 143.25 95.325) (end 143.25 93.675) (width 0.25) (layer "F.Cu") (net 3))
 (segment (start 143.25 93.364363) (end 144.759566 91.854797) (width 0.25) (layer "F.Cu") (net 3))
 (segment (start 143.425 95.5) (end 143.25 95.325) (width 0.25) (layer "F.Cu") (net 3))
 (via (at 143.25 93.675) (size 0.8) (drill 0.4) (layers "F.Cu" "B.Cu") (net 3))
 (segment (start 143.25 93.675) (end 143.25 91.795) (width 0.25) (layer "B.Cu") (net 3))
 (segment (start 143.25 91.795) (end 142.845 91.39) (width 0.25) (layer "B.Cu") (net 3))
 (segment (start 158.1 94.95) (end 157.125 93.975) (width 0.25) (layer "F.Cu") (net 12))
 (segment (start 157.125 93.975) (end 157.075 93.975) (width 0.25) (layer "F.Cu") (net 12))
 (via (at 157.075 93.975) (size 0.8) (drill 0.4) (layers "F.Cu" "B.Cu") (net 12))
 (segment (start 154.8 91.7) (end 157.075 93.975) (width 0.25) (layer "B.Cu") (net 12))
 (segment (start 154.3 91.7) (end 154.8 91.7) (width 0.25) (layer "B.Cu") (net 12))
 (segment (start 139.525 94.127669) (end 141.797872 91.854797) (width 0.25) (layer "F.Cu") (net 2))
 (segment (start 139.525 94.95) (end 139.525 94.127669) (width 0.25) (layer "F.Cu") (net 2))
 (segment (start 138.99 98.685) (end 138.99 100.2875) (width 0.25) (layer "F.Cu") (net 13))
 (segment (start 139.8 97.875) (end 138.99 98.685) (width 0.25) (layer "F.Cu") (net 13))
 (segment (start 138.99 100.2875) (end 138.99 98.69) (width 0.25) (layer "F.Cu") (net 13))
 (segment (start 138.99 98.69) (end 137.075 96.775) (width 0.25) (layer "F.Cu") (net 13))
 (segment (start 142.5 97.575) (end 141 97.575) (width 0.25) (layer "F.Cu") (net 13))
 (segment (start 140.7 97.875) (end 139.8 97.875) (width 0.25) (layer "F.Cu") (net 13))
 (segment (start 141 97.575) (end 140.7 97.875) (width 0.25) (layer "F.Cu") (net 13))
 (via (at 142.5 97.575) (size 0.8) (drill 0.4) (layers "F.Cu" "B.Cu") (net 13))
 (segment (start 142.845 99.01) (end 142.845 97.92) (width 0.25) (layer "B.Cu") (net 13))
 (segment (start 142.845 97.92) (end 142.5 97.575) (width 0.25) (layer "B.Cu") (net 13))
 (segment (start 147.325 96.775) (end 147.325 100.2625) (width 0.25) (layer "F.Cu") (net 9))
 (segment (start 147.325 100.2625) (end 147.3 100.2875) (width 0.25) (layer "F.Cu") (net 9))
 (segment (start 137.881382 90.9) (end 136.6 90.9) (width 0.25) (layer "F.Cu") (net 1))
 (segment (start 138.836179 91.854797) (end 137.881382 90.9) (width 0.25) (layer "F.Cu") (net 1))
 (segment (start 149.05 90.9) (end 147.8 90.9) (width 0.25) (layer "F.Cu") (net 14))
 (segment (start 150.025 91.875) (end 149.05 90.9) (width 0.25) (layer "F.Cu") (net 14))
 (segment (start 146.825 94) (end 146.825 94.45) (width 0.25) (layer "F.Cu") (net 10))
 (segment (start 146.825 94.45) (end 147.325 94.95) (width 0.25) (layer "F.Cu") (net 10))
 (via (at 146.825 94) (size 0.8) (drill 0.4) (layers "F.Cu" "B.Cu") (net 10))
 (segment (start 148.1 93.6) (end 147.225 93.6) (width 0.25) (layer "B.Cu") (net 10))
 (segment (start 147.225 93.6) (end 146.825 94) (width 0.25) (layer "B.Cu") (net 10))
 (segment (start 149.7 93.975) (end 149.7 94.71) (width 0.25) (layer "F.Cu") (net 11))
 (segment (start 149.7 94.71) (end 149.46 94.95) (width 0.25) (layer "F.Cu") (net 11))
 (via (at 149.7 93.975) (size 0.8) (drill 0.4) (layers "F.Cu" "B.Cu") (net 11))
 (segment (start 149.975 93.7) (end 149.7 93.975) (width 0.25) (layer "B.Cu") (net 11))
 (segment (start 149.975 92.65) (end 149.975 93.7) (width 0.25) (layer "B.Cu") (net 11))
 (segment (start 152.425 92.65) (end 149.975 92.65) (width 0.25) (layer "B.Cu") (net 11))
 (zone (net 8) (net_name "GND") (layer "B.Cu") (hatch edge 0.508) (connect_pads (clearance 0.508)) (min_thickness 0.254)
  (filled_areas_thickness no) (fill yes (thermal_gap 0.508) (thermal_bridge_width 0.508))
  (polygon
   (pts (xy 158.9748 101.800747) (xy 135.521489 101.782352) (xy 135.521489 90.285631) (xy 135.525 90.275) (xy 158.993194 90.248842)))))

